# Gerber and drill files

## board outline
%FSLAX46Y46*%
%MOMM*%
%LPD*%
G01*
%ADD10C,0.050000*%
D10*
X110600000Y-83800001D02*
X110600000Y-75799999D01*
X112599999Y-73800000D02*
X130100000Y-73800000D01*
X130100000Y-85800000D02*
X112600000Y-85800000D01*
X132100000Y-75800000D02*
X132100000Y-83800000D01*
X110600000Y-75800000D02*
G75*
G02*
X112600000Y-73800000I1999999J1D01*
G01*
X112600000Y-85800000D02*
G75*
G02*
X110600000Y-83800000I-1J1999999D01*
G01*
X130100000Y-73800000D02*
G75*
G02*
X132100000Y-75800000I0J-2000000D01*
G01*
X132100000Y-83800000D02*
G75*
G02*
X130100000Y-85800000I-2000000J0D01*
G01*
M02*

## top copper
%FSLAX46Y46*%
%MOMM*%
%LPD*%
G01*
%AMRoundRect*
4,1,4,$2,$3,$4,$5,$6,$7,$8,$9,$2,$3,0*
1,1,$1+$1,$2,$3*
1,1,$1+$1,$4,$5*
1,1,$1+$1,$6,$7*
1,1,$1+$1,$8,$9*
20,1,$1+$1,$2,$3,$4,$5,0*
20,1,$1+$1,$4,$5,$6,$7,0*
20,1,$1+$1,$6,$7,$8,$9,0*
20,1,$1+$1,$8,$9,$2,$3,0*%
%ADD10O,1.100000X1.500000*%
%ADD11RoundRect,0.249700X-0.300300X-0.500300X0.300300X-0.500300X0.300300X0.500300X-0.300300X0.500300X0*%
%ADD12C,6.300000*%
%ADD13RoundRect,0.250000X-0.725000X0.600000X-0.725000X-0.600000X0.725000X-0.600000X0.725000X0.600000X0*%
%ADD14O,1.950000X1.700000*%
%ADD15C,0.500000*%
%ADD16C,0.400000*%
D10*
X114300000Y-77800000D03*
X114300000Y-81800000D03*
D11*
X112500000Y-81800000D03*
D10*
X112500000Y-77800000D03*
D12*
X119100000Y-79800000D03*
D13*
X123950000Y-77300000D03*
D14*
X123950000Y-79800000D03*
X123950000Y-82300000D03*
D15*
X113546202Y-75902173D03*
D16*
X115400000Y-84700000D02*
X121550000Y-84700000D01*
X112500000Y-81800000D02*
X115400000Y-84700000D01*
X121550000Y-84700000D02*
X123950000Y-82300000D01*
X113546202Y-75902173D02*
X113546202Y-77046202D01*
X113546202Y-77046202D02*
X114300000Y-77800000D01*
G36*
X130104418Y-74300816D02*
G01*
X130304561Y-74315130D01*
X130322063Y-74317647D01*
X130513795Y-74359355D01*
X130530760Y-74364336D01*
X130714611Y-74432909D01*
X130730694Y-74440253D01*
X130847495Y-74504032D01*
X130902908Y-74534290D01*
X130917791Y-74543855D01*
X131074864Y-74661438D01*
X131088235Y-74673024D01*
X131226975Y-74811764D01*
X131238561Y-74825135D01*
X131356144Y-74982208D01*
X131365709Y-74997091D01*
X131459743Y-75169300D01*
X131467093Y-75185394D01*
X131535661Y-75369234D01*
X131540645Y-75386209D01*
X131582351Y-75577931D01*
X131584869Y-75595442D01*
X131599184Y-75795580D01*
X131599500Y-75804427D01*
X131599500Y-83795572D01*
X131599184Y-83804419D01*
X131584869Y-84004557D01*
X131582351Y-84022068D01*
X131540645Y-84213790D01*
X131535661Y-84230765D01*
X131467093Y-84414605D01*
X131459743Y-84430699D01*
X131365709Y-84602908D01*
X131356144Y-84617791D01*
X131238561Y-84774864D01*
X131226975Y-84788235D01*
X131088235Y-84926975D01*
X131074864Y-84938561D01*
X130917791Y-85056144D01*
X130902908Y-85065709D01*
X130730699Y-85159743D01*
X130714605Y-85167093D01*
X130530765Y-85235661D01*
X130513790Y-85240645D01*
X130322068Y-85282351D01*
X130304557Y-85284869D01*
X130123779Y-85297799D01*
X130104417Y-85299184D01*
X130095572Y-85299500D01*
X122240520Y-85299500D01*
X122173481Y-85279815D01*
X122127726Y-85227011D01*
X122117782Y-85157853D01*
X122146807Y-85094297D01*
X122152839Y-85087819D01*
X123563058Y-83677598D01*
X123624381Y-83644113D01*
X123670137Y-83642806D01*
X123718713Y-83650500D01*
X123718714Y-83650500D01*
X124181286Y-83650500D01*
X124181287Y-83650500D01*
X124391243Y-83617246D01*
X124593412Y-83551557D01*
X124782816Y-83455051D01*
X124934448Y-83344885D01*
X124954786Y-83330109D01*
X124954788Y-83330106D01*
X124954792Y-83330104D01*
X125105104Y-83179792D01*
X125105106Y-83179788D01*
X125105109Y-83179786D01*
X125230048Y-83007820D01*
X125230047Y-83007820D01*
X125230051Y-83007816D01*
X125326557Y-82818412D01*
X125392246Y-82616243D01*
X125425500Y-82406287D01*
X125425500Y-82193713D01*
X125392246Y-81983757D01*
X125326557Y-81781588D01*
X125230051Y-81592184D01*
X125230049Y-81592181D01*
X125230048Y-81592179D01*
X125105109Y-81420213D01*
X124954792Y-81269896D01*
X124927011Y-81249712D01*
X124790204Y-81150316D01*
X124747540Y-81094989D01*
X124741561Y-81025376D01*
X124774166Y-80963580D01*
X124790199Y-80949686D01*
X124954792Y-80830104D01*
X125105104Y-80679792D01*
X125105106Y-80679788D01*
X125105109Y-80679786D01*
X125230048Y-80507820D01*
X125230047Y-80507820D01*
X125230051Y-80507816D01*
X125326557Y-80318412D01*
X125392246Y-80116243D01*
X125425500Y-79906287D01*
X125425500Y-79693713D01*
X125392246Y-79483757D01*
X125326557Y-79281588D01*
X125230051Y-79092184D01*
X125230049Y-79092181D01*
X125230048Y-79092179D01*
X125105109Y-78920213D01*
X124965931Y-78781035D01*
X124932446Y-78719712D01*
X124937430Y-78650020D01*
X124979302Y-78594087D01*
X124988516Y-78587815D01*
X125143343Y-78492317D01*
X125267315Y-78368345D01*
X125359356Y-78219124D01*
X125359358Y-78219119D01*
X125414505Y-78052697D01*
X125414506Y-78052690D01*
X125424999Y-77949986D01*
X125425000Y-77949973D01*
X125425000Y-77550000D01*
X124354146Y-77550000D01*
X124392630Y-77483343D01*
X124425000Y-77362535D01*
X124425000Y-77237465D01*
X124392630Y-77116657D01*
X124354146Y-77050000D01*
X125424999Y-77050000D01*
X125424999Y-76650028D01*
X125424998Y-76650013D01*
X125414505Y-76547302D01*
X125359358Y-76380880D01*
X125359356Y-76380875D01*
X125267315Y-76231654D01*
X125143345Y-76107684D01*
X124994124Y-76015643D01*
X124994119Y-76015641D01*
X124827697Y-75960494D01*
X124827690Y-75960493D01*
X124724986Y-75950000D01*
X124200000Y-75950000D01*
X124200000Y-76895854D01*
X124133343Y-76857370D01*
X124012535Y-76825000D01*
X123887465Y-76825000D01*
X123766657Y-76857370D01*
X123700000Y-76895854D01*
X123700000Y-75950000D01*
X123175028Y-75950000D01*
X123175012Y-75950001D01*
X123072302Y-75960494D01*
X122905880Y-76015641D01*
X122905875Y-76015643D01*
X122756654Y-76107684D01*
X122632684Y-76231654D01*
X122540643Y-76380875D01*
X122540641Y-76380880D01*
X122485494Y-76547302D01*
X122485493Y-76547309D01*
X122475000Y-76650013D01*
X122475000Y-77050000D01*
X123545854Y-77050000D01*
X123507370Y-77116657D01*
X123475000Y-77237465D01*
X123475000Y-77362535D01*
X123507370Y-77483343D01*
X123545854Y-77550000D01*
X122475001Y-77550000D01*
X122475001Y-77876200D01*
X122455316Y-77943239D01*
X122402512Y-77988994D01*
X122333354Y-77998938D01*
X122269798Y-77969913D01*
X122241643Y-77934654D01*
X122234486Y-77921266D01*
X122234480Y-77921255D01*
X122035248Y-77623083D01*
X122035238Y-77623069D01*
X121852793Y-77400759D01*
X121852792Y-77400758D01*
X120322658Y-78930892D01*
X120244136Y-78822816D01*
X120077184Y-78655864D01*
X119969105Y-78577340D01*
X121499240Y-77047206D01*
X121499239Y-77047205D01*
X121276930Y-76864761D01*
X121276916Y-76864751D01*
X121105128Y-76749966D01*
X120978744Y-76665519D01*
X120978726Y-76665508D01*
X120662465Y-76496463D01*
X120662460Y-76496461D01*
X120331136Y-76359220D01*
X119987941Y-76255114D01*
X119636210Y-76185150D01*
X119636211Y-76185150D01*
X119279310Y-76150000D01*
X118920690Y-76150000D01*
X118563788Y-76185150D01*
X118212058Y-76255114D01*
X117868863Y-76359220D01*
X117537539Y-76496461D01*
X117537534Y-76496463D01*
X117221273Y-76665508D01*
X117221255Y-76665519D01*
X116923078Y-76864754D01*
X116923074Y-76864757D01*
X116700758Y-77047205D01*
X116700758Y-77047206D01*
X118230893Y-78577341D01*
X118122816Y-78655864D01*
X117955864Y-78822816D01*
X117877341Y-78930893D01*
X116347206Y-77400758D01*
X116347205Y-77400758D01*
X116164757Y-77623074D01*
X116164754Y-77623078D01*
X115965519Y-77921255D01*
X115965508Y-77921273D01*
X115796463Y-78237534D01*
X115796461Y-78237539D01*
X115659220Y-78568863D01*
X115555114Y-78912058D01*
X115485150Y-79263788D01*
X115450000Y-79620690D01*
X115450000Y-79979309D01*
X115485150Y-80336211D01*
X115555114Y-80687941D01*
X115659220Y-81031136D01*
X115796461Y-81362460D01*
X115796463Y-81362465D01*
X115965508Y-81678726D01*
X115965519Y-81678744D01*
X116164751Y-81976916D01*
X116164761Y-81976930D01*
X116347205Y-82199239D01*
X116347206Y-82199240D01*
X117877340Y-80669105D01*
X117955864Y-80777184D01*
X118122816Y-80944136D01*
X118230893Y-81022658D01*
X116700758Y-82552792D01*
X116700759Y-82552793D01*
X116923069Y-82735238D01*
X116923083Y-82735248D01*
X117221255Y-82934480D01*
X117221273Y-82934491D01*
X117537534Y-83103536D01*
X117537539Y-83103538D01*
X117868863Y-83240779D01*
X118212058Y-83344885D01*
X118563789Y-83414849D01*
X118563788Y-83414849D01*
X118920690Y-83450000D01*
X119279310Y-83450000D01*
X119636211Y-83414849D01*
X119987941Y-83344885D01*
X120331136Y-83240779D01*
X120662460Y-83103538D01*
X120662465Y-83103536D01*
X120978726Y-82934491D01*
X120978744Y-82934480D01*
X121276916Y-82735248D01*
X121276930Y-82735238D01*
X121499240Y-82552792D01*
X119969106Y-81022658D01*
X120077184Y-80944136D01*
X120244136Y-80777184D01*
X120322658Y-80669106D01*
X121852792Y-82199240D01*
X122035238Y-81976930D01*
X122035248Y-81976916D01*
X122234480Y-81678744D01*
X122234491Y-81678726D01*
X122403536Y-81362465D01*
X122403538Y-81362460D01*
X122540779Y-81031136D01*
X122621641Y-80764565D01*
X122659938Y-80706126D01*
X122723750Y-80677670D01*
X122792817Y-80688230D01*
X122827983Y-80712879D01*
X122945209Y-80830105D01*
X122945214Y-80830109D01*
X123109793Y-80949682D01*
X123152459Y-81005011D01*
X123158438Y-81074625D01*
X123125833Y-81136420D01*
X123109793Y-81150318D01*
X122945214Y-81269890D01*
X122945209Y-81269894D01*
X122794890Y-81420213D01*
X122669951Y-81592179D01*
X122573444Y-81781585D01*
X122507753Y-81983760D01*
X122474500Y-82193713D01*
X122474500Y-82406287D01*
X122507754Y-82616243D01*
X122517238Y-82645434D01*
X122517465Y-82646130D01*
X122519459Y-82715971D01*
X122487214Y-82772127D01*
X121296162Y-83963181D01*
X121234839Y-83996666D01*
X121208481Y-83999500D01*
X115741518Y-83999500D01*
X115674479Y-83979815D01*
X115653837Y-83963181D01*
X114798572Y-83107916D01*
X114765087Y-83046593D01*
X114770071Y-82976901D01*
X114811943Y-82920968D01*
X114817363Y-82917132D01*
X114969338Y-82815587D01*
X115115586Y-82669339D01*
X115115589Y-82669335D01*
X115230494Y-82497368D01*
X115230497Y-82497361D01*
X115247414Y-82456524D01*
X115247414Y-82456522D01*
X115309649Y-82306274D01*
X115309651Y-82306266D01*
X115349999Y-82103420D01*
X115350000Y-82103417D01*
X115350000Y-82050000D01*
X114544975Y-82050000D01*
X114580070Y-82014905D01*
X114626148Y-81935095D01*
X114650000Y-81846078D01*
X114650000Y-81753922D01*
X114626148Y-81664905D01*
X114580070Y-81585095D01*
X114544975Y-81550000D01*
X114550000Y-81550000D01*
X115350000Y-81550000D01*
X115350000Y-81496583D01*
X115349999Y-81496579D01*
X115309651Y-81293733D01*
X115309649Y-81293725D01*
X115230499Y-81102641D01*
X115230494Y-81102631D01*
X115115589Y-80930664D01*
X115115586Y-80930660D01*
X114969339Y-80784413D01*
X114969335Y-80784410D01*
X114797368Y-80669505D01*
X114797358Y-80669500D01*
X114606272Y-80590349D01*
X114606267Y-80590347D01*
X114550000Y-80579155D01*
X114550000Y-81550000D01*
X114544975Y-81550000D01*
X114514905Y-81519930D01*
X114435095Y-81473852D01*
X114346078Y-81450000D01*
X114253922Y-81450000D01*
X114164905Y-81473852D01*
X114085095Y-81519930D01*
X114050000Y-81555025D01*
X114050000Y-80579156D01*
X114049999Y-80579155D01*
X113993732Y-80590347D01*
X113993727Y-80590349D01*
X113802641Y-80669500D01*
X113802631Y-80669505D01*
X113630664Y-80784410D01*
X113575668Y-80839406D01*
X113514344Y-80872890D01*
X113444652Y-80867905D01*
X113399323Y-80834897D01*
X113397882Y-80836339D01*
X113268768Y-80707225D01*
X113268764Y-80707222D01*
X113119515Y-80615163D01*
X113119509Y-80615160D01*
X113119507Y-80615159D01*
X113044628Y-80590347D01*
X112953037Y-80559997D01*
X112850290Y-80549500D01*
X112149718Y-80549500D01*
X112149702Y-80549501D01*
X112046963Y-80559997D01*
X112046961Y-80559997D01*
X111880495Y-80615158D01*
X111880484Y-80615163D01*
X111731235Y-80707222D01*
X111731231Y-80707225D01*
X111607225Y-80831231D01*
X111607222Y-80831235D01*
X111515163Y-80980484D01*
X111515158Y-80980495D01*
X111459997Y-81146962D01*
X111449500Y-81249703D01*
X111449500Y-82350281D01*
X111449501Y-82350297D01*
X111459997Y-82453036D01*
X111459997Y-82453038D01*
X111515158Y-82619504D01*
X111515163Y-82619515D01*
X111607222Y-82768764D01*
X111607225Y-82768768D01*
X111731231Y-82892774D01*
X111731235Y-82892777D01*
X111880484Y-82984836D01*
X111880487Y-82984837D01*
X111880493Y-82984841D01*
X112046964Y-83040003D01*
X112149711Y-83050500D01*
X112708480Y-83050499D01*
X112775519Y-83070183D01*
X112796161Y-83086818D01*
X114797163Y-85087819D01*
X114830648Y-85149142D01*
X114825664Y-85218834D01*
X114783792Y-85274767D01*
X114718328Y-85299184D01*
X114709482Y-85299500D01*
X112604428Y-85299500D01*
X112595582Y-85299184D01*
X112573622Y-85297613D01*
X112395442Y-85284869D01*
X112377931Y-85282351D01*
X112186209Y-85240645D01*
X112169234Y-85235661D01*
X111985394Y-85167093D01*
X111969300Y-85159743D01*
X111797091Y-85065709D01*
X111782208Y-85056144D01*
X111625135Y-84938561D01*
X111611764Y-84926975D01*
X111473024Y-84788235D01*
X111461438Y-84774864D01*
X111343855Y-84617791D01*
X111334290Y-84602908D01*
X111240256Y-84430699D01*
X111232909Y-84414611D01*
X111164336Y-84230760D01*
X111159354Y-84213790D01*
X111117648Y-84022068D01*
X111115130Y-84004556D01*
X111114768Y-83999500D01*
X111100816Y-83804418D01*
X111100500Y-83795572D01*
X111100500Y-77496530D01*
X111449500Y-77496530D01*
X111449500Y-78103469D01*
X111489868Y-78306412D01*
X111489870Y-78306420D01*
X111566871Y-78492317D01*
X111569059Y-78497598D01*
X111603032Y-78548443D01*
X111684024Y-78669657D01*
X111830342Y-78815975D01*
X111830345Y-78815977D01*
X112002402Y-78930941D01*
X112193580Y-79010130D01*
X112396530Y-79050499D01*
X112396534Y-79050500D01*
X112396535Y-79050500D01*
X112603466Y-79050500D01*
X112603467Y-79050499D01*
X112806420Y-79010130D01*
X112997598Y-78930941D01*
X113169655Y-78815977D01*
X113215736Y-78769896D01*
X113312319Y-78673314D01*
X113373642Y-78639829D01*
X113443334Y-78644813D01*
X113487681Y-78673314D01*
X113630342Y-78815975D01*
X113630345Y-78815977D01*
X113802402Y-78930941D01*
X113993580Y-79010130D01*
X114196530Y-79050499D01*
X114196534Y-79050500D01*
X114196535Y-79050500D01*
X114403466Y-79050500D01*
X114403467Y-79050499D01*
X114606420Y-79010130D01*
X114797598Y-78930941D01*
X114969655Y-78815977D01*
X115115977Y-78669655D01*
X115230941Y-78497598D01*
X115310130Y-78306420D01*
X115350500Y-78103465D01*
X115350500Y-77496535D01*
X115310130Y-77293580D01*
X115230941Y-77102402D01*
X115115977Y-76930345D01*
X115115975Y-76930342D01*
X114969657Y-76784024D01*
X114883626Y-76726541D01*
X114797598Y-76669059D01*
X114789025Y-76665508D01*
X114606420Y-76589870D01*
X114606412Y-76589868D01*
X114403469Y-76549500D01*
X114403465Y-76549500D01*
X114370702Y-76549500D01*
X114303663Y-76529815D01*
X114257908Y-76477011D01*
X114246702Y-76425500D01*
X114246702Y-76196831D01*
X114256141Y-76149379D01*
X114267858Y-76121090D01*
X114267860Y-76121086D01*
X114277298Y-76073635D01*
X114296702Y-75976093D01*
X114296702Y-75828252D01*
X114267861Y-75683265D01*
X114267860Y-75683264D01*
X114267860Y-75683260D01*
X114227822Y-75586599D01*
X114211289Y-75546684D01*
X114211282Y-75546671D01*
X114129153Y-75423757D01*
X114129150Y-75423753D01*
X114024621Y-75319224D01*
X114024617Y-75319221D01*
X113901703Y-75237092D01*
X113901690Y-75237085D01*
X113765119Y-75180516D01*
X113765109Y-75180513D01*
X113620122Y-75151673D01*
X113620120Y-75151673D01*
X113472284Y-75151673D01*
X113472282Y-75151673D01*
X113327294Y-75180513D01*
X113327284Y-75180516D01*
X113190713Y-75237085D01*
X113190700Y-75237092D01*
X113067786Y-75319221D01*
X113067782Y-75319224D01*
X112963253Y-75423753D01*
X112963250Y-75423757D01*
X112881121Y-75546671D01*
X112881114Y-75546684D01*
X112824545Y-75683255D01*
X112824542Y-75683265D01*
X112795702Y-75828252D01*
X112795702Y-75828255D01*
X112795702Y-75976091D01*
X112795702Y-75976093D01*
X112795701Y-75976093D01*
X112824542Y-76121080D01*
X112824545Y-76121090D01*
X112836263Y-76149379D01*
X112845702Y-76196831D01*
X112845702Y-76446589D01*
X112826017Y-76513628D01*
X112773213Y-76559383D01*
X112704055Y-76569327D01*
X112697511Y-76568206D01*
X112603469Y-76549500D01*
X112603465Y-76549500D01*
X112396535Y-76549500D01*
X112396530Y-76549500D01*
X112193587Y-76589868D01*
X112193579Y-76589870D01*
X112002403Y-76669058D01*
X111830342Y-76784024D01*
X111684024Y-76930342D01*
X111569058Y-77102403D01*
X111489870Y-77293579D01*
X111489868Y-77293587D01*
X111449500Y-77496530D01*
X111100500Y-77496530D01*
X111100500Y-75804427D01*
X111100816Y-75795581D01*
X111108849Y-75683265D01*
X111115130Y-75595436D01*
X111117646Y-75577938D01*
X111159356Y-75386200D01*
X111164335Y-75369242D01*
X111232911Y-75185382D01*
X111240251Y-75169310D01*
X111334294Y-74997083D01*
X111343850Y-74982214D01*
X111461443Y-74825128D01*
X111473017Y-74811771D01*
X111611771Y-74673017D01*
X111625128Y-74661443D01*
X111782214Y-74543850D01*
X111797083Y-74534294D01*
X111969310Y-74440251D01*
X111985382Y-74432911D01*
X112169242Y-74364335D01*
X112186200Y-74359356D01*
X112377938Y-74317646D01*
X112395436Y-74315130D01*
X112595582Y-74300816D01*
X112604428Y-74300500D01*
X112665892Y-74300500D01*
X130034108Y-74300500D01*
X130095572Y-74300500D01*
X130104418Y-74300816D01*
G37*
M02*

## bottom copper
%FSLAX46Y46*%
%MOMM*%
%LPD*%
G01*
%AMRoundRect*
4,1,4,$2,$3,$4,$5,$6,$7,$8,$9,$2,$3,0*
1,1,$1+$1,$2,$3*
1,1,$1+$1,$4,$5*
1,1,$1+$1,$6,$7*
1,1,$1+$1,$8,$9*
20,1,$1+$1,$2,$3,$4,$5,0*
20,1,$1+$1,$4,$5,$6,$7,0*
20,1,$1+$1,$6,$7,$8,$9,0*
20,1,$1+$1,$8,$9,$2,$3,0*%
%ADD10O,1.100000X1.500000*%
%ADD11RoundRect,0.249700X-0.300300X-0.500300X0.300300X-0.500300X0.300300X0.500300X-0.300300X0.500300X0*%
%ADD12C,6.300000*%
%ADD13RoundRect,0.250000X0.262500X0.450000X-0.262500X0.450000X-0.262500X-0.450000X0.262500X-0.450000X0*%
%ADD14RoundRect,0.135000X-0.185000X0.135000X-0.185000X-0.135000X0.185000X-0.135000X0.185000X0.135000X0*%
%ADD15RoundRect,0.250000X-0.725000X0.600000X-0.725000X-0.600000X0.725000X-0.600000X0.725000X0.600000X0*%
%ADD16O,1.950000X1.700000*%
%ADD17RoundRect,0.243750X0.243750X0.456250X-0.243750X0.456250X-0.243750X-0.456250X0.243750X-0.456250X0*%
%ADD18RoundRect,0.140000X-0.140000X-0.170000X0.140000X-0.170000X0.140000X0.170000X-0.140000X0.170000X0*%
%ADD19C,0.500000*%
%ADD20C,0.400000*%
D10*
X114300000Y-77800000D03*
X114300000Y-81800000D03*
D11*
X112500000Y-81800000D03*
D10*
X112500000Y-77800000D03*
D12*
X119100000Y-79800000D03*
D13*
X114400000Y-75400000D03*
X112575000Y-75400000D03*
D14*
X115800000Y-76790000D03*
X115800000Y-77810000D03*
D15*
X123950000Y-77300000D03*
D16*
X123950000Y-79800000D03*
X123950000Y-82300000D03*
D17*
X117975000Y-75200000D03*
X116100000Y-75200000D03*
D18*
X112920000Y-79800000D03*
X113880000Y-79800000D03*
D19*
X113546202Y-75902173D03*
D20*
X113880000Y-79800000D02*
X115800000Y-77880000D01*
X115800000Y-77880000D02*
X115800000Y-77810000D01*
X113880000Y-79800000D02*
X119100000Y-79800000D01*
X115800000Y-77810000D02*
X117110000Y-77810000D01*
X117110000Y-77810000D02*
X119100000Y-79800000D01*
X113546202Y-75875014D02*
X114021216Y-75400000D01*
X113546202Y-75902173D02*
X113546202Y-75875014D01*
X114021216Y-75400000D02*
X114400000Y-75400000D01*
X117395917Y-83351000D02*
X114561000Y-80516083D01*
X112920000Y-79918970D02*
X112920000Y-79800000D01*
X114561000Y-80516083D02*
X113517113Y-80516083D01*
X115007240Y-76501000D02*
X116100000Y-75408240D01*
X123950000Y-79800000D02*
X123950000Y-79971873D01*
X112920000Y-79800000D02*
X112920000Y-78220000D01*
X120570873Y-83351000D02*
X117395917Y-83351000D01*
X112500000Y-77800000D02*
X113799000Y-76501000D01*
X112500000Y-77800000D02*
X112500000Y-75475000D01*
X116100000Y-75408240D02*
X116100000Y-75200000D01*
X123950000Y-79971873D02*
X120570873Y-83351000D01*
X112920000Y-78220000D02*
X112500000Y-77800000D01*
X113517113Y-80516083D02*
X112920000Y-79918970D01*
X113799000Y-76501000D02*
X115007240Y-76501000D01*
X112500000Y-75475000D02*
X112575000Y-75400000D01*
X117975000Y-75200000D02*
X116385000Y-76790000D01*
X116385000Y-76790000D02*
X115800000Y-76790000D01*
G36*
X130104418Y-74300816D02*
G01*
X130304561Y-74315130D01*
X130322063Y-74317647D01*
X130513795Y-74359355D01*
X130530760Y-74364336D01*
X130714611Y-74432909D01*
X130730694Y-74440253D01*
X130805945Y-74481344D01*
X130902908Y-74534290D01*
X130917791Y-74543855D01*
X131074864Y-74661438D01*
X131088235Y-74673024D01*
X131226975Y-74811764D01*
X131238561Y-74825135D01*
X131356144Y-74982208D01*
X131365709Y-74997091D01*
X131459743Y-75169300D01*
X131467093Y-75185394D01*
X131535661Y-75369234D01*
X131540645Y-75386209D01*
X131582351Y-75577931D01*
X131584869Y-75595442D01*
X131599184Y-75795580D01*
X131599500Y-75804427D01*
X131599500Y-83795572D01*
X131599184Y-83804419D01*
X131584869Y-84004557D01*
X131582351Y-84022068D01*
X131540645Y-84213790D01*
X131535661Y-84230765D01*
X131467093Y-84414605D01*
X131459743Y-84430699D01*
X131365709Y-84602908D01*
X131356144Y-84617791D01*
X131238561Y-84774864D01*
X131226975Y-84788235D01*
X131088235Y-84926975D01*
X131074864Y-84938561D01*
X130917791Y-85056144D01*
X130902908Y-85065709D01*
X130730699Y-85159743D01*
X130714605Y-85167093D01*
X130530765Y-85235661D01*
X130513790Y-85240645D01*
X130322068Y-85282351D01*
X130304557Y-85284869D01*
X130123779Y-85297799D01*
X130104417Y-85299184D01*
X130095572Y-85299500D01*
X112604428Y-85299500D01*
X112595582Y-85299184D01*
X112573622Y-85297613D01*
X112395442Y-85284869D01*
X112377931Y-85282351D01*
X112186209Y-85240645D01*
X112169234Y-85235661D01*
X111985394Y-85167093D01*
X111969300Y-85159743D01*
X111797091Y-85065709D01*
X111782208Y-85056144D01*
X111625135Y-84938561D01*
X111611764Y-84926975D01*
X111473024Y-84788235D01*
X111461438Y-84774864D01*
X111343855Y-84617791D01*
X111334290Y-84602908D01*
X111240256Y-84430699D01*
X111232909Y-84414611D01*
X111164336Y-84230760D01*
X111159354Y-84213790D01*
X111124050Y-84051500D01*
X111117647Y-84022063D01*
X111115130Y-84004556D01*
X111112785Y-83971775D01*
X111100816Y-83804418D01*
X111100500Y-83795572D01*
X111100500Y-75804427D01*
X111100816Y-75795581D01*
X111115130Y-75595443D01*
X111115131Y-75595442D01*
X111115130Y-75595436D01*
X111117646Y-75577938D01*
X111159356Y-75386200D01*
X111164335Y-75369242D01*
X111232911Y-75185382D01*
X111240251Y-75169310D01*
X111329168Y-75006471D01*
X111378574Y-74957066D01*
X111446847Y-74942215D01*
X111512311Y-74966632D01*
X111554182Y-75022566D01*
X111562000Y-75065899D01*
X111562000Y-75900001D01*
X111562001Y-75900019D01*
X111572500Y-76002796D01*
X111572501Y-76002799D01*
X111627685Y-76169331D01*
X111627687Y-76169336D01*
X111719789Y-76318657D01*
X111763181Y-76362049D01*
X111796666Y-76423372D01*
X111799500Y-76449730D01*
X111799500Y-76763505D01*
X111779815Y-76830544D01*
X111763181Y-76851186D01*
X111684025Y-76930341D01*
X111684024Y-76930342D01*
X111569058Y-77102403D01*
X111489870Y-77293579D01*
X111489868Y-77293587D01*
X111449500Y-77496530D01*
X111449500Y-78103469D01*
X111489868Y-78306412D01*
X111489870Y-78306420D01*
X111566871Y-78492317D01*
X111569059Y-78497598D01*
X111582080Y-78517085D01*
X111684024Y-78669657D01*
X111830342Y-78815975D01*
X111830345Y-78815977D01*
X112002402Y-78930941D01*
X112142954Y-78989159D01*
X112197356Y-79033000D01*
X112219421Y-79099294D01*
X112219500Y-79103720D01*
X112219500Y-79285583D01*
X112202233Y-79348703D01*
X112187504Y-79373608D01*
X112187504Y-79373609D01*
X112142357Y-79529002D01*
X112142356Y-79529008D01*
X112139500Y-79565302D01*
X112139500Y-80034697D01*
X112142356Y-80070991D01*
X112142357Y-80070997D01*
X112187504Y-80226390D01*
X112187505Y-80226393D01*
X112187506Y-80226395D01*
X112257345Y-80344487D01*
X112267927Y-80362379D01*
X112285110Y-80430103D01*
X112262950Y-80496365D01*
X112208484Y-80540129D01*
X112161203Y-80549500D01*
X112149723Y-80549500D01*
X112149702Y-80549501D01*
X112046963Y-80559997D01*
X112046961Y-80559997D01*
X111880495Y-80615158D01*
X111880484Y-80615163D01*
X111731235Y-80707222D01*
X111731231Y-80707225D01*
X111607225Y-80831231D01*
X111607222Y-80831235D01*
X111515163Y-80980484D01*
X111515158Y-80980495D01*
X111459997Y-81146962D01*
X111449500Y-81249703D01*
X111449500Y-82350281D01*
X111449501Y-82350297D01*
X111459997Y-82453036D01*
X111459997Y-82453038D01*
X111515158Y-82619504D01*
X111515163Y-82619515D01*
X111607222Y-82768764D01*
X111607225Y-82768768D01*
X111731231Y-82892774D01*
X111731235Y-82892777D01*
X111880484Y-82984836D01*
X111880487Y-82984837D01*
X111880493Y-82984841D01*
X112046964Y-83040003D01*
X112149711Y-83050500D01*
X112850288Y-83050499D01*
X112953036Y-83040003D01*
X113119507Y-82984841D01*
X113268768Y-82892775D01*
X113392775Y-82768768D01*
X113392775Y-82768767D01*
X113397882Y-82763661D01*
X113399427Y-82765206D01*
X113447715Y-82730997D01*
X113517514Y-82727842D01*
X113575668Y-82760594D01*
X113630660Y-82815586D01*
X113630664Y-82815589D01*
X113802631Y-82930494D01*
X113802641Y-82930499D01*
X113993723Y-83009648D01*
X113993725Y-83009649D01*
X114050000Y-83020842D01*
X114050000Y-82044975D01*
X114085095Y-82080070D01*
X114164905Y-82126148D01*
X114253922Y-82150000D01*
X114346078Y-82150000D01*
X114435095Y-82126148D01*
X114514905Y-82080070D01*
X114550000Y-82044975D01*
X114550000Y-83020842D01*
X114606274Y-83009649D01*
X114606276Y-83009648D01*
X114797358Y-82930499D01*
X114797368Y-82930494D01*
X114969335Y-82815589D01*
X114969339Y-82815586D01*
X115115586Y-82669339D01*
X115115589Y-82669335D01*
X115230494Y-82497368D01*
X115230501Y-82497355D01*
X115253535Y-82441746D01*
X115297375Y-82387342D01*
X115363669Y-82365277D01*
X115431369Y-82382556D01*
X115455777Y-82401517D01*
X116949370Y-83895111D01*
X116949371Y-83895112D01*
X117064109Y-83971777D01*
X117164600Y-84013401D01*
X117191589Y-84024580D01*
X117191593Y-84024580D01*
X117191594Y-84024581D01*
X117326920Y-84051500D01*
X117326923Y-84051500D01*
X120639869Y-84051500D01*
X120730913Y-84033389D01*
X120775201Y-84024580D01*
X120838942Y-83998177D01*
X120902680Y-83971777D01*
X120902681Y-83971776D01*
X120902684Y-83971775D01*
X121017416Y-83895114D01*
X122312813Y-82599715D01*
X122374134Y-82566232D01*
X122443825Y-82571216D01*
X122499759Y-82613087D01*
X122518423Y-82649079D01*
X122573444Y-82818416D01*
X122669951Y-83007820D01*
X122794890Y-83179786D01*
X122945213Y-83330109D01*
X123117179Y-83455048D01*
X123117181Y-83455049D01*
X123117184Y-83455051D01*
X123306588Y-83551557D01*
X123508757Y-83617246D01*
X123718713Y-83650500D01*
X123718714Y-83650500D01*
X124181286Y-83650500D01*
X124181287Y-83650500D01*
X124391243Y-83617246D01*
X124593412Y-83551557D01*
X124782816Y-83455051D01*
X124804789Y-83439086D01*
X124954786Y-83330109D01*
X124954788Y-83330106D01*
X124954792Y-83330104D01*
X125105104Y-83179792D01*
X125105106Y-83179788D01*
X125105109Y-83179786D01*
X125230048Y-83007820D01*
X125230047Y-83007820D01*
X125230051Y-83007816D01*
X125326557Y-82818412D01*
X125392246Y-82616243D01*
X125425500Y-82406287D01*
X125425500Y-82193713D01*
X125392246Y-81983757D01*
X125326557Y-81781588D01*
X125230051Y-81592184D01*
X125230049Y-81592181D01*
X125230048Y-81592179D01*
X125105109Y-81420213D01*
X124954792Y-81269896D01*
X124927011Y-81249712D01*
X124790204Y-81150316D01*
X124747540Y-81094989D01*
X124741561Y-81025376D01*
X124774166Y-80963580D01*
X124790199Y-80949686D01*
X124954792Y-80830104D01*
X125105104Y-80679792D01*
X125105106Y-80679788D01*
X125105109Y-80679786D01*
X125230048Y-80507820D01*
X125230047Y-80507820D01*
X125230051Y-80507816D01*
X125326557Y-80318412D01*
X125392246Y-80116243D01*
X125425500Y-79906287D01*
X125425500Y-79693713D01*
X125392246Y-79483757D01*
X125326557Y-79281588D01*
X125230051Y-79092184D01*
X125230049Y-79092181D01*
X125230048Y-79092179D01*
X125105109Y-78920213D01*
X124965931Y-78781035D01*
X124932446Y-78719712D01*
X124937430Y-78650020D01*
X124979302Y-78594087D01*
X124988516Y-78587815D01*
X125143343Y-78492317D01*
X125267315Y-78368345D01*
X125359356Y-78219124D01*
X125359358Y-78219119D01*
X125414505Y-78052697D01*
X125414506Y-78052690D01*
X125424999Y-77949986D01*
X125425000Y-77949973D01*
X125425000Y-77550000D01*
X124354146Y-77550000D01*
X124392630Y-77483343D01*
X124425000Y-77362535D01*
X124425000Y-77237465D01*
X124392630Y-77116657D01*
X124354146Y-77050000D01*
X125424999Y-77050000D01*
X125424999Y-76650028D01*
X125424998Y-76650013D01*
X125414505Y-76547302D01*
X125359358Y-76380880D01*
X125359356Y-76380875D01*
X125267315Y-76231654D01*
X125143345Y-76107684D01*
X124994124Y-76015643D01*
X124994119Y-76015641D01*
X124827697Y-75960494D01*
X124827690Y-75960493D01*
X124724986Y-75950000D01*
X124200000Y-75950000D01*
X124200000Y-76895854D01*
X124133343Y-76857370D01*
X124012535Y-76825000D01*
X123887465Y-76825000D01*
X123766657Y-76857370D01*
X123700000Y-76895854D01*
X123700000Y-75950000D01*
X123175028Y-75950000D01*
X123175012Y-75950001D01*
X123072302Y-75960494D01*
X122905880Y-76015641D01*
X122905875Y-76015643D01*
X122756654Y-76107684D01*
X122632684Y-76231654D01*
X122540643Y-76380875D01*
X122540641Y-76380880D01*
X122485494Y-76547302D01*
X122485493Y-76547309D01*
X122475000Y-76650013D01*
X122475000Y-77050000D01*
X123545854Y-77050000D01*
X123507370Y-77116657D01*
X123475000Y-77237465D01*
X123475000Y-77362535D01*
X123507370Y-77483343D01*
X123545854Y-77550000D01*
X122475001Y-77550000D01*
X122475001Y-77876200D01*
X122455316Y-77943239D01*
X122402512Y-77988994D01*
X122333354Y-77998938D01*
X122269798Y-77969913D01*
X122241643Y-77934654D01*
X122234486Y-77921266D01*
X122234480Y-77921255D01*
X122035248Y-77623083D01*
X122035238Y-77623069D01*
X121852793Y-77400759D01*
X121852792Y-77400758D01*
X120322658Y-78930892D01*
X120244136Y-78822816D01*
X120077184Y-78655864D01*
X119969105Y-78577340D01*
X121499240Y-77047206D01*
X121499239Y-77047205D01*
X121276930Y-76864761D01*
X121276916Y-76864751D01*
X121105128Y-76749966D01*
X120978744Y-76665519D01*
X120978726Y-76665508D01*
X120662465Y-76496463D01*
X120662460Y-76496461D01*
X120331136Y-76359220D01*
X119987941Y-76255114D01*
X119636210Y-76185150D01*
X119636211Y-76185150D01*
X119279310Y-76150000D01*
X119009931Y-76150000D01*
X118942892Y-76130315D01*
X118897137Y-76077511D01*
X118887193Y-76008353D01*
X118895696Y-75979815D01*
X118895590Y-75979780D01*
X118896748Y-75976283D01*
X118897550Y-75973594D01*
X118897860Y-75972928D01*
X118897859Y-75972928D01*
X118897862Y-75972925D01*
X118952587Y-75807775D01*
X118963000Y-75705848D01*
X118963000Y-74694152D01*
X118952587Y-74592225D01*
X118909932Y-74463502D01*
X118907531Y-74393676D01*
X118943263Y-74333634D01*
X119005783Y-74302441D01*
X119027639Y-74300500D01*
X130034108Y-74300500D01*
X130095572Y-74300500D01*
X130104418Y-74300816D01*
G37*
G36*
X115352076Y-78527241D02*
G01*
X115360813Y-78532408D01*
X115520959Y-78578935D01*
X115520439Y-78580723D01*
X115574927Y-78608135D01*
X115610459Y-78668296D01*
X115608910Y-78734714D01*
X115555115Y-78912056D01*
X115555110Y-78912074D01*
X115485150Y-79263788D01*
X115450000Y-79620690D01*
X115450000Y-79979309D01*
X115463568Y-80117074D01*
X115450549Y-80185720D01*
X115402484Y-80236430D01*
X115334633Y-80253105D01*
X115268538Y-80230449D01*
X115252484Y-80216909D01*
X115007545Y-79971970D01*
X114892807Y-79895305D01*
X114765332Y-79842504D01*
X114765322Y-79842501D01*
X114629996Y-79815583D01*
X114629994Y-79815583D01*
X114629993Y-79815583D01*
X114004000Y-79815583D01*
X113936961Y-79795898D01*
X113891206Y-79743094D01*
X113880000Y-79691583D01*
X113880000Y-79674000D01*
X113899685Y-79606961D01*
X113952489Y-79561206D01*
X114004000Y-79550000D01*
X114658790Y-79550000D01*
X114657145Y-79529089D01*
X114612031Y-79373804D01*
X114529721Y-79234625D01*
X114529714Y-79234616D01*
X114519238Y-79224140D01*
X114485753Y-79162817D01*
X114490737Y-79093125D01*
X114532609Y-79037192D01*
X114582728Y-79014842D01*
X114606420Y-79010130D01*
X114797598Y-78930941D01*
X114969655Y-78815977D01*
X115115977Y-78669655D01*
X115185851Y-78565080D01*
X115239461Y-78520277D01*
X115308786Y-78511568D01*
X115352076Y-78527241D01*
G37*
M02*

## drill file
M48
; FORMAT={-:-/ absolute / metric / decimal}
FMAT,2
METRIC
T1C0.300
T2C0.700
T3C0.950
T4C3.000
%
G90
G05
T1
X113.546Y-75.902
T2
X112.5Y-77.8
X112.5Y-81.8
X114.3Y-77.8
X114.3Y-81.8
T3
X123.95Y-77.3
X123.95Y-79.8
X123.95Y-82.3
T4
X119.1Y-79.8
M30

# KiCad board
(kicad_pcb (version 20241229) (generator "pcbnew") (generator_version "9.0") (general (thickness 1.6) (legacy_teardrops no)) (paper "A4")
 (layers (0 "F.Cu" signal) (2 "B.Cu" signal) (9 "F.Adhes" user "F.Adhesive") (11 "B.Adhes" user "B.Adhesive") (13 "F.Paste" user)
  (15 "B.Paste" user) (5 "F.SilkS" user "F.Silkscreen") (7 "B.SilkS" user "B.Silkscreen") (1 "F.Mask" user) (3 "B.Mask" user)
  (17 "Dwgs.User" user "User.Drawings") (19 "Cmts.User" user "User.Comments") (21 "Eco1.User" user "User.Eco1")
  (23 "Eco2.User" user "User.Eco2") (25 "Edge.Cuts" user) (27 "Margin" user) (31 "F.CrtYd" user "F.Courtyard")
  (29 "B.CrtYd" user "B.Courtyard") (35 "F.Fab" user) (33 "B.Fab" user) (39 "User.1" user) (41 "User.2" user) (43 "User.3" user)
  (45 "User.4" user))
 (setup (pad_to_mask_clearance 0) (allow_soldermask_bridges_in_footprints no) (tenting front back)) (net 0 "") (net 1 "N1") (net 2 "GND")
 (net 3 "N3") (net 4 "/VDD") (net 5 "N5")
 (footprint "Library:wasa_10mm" (layer "F.Cu") (at 124.3 84.4)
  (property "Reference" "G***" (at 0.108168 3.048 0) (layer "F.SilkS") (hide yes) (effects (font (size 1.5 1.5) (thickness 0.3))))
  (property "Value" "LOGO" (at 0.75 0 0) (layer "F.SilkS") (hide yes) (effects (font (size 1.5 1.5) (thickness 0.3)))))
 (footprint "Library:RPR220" (layer "F.Cu") (at 112.5 81.8)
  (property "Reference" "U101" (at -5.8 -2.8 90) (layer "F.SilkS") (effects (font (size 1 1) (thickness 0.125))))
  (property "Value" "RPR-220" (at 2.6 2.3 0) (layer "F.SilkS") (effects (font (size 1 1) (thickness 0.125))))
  (pad "1" thru_hole oval (at 1.8 -4) (size 1.1 1.5) (drill 0.7) (layers "*.Cu" "*.Mask") (remove_unused_layers no) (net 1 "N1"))
  (pad "2" thru_hole oval (at 1.8 0) (size 1.1 1.5) (drill 0.7) (layers "*.Cu" "*.Mask") (remove_unused_layers no) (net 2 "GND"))
  (pad "3" thru_hole roundrect (at 0 0) (size 1.1 1.5) (drill 0.7) (layers "*.Cu" "*.Mask") (remove_unused_layers no)
   (roundrect_rratio 0.227) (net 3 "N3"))
  (pad "4" thru_hole oval (at 0 -4) (size 1.1 1.5) (drill 0.7) (layers "*.Cu" "*.Mask") (remove_unused_layers no) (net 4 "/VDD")))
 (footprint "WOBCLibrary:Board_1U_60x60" (layer "F.Cu") (at 120.1 79.8)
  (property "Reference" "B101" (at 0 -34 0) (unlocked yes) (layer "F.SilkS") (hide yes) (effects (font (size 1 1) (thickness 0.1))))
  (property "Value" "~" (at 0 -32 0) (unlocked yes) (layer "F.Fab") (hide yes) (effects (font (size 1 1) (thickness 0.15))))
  (fp_line (start -9.5 4.000001) (end -9.5 -4.000001) (stroke (width 0.05) (type default)) (layer "Edge.Cuts"))
  (fp_line (start -7.500001 -6) (end 10 -6) (stroke (width 0.05) (type default)) (layer "Edge.Cuts"))
  (fp_line (start 10 6) (end -7.5 6) (stroke (width 0.05) (type default)) (layer "Edge.Cuts"))
  (fp_line (start 12 -4) (end 12 4) (stroke (width 0.05) (type default)) (layer "Edge.Cuts"))
  (fp_arc (start -9.5 -4) (mid -8.914214 -5.414214) (end -7.5 -6) (stroke (width 0.05) (type default)) (layer "Edge.Cuts"))
  (fp_arc (start -7.5 6) (mid -8.914214 5.414214) (end -9.5 4) (stroke (width 0.05) (type default)) (layer "Edge.Cuts"))
  (fp_arc (start 10 -6) (mid 11.414214 -5.414214) (end 12 -4) (stroke (width 0.05) (type default)) (layer "Edge.Cuts"))
  (fp_arc (start 12 4) (mid 11.414214 5.414214) (end 10 6) (stroke (width 0.05) (type default)) (layer "Edge.Cuts"))
  (pad "GND" thru_hole circle (at -1 0) (size 6.3 6.3) (drill 3) (layers "*.Cu" "*.Mask") (remove_unused_layers no) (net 2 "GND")))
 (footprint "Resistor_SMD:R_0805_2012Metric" (layer "B.Cu") (at 113.4875 75.4 180)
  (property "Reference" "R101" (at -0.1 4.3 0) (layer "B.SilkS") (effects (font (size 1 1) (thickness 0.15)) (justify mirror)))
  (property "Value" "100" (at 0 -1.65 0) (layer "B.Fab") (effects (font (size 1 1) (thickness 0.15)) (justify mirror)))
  (pad "1" smd roundrect (at -0.9125 0 180) (size 1.025 1.4) (layers "B.Cu" "B.Mask" "B.Paste") (roundrect_rratio 0.243902) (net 1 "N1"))
  (pad "2" smd roundrect (at 0.9125 0 180) (size 1.025 1.4) (layers "B.Cu" "B.Mask" "B.Paste") (roundrect_rratio 0.243902) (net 4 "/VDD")))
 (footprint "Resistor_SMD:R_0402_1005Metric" (layer "B.Cu") (at 115.8 77.3 -90)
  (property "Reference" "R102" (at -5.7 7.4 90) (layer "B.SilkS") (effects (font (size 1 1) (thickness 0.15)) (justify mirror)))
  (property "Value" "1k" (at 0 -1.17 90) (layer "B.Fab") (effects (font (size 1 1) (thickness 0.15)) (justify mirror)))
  (pad "1" smd roundrect (at -0.51 0 270) (size 0.54 0.64) (layers "B.Cu" "B.Mask" "B.Paste") (roundrect_rratio 0.25) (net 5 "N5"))
  (pad "2" smd roundrect (at 0.51 0 270) (size 0.54 0.64) (layers "B.Cu" "B.Mask" "B.Paste") (roundrect_rratio 0.25) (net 2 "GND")))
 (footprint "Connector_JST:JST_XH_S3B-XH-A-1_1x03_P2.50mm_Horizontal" (layer "B.Cu") (at 123.95 77.3 -90)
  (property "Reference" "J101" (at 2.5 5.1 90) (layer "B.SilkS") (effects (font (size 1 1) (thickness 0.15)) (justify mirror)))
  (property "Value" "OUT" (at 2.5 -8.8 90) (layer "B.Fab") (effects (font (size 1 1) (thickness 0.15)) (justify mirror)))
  (pad "1" thru_hole roundrect (at 0 0 270) (size 1.7 1.95) (drill 0.95) (layers "*.Cu" "*.Mask") (remove_unused_layers no)
   (roundrect_rratio 0.147059) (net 2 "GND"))
  (pad "2" thru_hole oval (at 2.5 0 270) (size 1.7 1.95) (drill 0.95) (layers "*.Cu" "*.Mask") (remove_unused_layers no) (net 4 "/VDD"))
  (pad "3" thru_hole oval (at 5 0 270) (size 1.7 1.95) (drill 0.95) (layers "*.Cu" "*.Mask") (remove_unused_layers no) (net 3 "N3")))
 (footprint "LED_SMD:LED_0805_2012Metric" (layer "B.Cu") (at 117.0375 75.2 180)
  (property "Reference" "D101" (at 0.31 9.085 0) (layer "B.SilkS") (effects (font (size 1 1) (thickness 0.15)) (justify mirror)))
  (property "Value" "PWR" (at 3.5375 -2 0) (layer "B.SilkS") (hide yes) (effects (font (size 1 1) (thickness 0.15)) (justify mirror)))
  (pad "1" smd roundrect (at -0.9375 0 180) (size 0.975 1.4) (layers "B.Cu" "B.Mask" "B.Paste") (roundrect_rratio 0.25) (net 5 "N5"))
  (pad "2" smd roundrect (at 0.9375 0 180) (size 0.975 1.4) (layers "B.Cu" "B.Mask" "B.Paste") (roundrect_rratio 0.25) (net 4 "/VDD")))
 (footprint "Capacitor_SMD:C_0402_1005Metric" (layer "B.Cu") (at 113.4 79.8)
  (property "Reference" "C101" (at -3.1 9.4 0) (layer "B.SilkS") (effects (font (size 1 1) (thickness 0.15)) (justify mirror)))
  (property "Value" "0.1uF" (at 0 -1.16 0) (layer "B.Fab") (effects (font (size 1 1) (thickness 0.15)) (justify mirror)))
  (pad "1" smd roundrect (at -0.48 0) (size 0.56 0.62) (layers "B.Cu" "B.Mask" "B.Paste") (roundrect_rratio 0.25) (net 4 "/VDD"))
  (pad "2" smd roundrect (at 0.48 0) (size 0.56 0.62) (layers "B.Cu" "B.Mask" "B.Paste") (roundrect_rratio 0.25) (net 2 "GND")))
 (segment (start 113.88 79.8) (end 115.8 77.88) (width 0.4) (layer "B.Cu") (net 2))
 (segment (start 115.8 77.88) (end 115.8 77.81) (width 0.4) (layer "B.Cu") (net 2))
 (segment (start 113.88 79.8) (end 119.1 79.8) (width 0.4) (layer "B.Cu") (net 2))
 (segment (start 115.8 77.81) (end 117.11 77.81) (width 0.4) (layer "B.Cu") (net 2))
 (segment (start 117.11 77.81) (end 119.1 79.8) (width 0.4) (layer "B.Cu") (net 2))
 (segment (start 115.4 84.7) (end 121.55 84.7) (width 0.4) (layer "F.Cu") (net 3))
 (segment (start 112.5 81.8) (end 115.4 84.7) (width 0.4) (layer "F.Cu") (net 3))
 (segment (start 121.55 84.7) (end 123.95 82.3) (width 0.4) (layer "F.Cu") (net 3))
 (segment (start 113.546202 75.902173) (end 113.546202 77.046202) (width 0.4) (layer "F.Cu") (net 1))
 (segment (start 113.546202 77.046202) (end 114.3 77.8) (width 0.4) (layer "F.Cu") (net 1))
 (via (at 113.546202 75.902173) (size 0.5) (drill 0.3) (layers "F.Cu" "B.Cu") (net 1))
 (segment (start 113.546202 75.875014) (end 114.021216 75.4) (width 0.4) (layer "B.Cu") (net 1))
 (segment (start 113.546202 75.902173) (end 113.546202 75.875014) (width 0.4) (layer "B.Cu") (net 1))
 (segment (start 114.021216 75.4) (end 114.4 75.4) (width 0.4) (layer "B.Cu") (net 1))
 (segment (start 117.395917 83.351) (end 114.561 80.516083) (width 0.4) (layer "B.Cu") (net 4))
 (segment (start 112.92 79.91897) (end 112.92 79.8) (width 0.4) (layer "B.Cu") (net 4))
 (segment (start 114.561 80.516083) (end 113.517113 80.516083) (width 0.4) (layer "B.Cu") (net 4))
 (segment (start 115.00724 76.501) (end 116.1 75.40824) (width 0.4) (layer "B.Cu") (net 4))
 (segment (start 123.95 79.8) (end 123.95 79.971873) (width 0.4) (layer "B.Cu") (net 4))
 (segment (start 112.92 79.8) (end 112.92 78.22) (width 0.4) (layer "B.Cu") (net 4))
 (segment (start 120.570873 83.351) (end 117.395917 83.351) (width 0.4) (layer "B.Cu") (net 4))
 (segment (start 112.5 77.8) (end 113.799 76.501) (width 0.4) (layer "B.Cu") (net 4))
 (segment (start 112.5 77.8) (end 112.5 75.475) (width 0.4) (layer "B.Cu") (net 4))
 (segment (start 116.1 75.40824) (end 116.1 75.2) (width 0.4) (layer "B.Cu") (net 4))
 (segment (start 123.95 79.971873) (end 120.570873 83.351) (width 0.4) (layer "B.Cu") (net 4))
 (segment (start 112.92 78.22) (end 112.5 77.8) (width 0.4) (layer "B.Cu") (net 4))
 (segment (start 113.517113 80.516083) (end 112.92 79.91897) (width 0.4) (layer "B.Cu") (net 4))
 (segment (start 113.799 76.501) (end 115.00724 76.501) (width 0.4) (layer "B.Cu") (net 4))
 (segment (start 112.5 75.475) (end 112.575 75.4) (width 0.4) (layer "B.Cu") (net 4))
 (segment (start 117.975 75.2) (end 116.385 76.79) (width 0.4) (layer "B.Cu") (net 5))
 (segment (start 116.385 76.79) (end 115.8 76.79) (width 0.4) (layer "B.Cu") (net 5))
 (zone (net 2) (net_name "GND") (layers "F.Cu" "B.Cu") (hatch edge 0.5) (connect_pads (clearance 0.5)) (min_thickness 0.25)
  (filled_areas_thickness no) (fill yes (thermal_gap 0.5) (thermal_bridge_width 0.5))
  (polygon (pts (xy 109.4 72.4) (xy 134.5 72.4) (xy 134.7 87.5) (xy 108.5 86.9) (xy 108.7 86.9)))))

